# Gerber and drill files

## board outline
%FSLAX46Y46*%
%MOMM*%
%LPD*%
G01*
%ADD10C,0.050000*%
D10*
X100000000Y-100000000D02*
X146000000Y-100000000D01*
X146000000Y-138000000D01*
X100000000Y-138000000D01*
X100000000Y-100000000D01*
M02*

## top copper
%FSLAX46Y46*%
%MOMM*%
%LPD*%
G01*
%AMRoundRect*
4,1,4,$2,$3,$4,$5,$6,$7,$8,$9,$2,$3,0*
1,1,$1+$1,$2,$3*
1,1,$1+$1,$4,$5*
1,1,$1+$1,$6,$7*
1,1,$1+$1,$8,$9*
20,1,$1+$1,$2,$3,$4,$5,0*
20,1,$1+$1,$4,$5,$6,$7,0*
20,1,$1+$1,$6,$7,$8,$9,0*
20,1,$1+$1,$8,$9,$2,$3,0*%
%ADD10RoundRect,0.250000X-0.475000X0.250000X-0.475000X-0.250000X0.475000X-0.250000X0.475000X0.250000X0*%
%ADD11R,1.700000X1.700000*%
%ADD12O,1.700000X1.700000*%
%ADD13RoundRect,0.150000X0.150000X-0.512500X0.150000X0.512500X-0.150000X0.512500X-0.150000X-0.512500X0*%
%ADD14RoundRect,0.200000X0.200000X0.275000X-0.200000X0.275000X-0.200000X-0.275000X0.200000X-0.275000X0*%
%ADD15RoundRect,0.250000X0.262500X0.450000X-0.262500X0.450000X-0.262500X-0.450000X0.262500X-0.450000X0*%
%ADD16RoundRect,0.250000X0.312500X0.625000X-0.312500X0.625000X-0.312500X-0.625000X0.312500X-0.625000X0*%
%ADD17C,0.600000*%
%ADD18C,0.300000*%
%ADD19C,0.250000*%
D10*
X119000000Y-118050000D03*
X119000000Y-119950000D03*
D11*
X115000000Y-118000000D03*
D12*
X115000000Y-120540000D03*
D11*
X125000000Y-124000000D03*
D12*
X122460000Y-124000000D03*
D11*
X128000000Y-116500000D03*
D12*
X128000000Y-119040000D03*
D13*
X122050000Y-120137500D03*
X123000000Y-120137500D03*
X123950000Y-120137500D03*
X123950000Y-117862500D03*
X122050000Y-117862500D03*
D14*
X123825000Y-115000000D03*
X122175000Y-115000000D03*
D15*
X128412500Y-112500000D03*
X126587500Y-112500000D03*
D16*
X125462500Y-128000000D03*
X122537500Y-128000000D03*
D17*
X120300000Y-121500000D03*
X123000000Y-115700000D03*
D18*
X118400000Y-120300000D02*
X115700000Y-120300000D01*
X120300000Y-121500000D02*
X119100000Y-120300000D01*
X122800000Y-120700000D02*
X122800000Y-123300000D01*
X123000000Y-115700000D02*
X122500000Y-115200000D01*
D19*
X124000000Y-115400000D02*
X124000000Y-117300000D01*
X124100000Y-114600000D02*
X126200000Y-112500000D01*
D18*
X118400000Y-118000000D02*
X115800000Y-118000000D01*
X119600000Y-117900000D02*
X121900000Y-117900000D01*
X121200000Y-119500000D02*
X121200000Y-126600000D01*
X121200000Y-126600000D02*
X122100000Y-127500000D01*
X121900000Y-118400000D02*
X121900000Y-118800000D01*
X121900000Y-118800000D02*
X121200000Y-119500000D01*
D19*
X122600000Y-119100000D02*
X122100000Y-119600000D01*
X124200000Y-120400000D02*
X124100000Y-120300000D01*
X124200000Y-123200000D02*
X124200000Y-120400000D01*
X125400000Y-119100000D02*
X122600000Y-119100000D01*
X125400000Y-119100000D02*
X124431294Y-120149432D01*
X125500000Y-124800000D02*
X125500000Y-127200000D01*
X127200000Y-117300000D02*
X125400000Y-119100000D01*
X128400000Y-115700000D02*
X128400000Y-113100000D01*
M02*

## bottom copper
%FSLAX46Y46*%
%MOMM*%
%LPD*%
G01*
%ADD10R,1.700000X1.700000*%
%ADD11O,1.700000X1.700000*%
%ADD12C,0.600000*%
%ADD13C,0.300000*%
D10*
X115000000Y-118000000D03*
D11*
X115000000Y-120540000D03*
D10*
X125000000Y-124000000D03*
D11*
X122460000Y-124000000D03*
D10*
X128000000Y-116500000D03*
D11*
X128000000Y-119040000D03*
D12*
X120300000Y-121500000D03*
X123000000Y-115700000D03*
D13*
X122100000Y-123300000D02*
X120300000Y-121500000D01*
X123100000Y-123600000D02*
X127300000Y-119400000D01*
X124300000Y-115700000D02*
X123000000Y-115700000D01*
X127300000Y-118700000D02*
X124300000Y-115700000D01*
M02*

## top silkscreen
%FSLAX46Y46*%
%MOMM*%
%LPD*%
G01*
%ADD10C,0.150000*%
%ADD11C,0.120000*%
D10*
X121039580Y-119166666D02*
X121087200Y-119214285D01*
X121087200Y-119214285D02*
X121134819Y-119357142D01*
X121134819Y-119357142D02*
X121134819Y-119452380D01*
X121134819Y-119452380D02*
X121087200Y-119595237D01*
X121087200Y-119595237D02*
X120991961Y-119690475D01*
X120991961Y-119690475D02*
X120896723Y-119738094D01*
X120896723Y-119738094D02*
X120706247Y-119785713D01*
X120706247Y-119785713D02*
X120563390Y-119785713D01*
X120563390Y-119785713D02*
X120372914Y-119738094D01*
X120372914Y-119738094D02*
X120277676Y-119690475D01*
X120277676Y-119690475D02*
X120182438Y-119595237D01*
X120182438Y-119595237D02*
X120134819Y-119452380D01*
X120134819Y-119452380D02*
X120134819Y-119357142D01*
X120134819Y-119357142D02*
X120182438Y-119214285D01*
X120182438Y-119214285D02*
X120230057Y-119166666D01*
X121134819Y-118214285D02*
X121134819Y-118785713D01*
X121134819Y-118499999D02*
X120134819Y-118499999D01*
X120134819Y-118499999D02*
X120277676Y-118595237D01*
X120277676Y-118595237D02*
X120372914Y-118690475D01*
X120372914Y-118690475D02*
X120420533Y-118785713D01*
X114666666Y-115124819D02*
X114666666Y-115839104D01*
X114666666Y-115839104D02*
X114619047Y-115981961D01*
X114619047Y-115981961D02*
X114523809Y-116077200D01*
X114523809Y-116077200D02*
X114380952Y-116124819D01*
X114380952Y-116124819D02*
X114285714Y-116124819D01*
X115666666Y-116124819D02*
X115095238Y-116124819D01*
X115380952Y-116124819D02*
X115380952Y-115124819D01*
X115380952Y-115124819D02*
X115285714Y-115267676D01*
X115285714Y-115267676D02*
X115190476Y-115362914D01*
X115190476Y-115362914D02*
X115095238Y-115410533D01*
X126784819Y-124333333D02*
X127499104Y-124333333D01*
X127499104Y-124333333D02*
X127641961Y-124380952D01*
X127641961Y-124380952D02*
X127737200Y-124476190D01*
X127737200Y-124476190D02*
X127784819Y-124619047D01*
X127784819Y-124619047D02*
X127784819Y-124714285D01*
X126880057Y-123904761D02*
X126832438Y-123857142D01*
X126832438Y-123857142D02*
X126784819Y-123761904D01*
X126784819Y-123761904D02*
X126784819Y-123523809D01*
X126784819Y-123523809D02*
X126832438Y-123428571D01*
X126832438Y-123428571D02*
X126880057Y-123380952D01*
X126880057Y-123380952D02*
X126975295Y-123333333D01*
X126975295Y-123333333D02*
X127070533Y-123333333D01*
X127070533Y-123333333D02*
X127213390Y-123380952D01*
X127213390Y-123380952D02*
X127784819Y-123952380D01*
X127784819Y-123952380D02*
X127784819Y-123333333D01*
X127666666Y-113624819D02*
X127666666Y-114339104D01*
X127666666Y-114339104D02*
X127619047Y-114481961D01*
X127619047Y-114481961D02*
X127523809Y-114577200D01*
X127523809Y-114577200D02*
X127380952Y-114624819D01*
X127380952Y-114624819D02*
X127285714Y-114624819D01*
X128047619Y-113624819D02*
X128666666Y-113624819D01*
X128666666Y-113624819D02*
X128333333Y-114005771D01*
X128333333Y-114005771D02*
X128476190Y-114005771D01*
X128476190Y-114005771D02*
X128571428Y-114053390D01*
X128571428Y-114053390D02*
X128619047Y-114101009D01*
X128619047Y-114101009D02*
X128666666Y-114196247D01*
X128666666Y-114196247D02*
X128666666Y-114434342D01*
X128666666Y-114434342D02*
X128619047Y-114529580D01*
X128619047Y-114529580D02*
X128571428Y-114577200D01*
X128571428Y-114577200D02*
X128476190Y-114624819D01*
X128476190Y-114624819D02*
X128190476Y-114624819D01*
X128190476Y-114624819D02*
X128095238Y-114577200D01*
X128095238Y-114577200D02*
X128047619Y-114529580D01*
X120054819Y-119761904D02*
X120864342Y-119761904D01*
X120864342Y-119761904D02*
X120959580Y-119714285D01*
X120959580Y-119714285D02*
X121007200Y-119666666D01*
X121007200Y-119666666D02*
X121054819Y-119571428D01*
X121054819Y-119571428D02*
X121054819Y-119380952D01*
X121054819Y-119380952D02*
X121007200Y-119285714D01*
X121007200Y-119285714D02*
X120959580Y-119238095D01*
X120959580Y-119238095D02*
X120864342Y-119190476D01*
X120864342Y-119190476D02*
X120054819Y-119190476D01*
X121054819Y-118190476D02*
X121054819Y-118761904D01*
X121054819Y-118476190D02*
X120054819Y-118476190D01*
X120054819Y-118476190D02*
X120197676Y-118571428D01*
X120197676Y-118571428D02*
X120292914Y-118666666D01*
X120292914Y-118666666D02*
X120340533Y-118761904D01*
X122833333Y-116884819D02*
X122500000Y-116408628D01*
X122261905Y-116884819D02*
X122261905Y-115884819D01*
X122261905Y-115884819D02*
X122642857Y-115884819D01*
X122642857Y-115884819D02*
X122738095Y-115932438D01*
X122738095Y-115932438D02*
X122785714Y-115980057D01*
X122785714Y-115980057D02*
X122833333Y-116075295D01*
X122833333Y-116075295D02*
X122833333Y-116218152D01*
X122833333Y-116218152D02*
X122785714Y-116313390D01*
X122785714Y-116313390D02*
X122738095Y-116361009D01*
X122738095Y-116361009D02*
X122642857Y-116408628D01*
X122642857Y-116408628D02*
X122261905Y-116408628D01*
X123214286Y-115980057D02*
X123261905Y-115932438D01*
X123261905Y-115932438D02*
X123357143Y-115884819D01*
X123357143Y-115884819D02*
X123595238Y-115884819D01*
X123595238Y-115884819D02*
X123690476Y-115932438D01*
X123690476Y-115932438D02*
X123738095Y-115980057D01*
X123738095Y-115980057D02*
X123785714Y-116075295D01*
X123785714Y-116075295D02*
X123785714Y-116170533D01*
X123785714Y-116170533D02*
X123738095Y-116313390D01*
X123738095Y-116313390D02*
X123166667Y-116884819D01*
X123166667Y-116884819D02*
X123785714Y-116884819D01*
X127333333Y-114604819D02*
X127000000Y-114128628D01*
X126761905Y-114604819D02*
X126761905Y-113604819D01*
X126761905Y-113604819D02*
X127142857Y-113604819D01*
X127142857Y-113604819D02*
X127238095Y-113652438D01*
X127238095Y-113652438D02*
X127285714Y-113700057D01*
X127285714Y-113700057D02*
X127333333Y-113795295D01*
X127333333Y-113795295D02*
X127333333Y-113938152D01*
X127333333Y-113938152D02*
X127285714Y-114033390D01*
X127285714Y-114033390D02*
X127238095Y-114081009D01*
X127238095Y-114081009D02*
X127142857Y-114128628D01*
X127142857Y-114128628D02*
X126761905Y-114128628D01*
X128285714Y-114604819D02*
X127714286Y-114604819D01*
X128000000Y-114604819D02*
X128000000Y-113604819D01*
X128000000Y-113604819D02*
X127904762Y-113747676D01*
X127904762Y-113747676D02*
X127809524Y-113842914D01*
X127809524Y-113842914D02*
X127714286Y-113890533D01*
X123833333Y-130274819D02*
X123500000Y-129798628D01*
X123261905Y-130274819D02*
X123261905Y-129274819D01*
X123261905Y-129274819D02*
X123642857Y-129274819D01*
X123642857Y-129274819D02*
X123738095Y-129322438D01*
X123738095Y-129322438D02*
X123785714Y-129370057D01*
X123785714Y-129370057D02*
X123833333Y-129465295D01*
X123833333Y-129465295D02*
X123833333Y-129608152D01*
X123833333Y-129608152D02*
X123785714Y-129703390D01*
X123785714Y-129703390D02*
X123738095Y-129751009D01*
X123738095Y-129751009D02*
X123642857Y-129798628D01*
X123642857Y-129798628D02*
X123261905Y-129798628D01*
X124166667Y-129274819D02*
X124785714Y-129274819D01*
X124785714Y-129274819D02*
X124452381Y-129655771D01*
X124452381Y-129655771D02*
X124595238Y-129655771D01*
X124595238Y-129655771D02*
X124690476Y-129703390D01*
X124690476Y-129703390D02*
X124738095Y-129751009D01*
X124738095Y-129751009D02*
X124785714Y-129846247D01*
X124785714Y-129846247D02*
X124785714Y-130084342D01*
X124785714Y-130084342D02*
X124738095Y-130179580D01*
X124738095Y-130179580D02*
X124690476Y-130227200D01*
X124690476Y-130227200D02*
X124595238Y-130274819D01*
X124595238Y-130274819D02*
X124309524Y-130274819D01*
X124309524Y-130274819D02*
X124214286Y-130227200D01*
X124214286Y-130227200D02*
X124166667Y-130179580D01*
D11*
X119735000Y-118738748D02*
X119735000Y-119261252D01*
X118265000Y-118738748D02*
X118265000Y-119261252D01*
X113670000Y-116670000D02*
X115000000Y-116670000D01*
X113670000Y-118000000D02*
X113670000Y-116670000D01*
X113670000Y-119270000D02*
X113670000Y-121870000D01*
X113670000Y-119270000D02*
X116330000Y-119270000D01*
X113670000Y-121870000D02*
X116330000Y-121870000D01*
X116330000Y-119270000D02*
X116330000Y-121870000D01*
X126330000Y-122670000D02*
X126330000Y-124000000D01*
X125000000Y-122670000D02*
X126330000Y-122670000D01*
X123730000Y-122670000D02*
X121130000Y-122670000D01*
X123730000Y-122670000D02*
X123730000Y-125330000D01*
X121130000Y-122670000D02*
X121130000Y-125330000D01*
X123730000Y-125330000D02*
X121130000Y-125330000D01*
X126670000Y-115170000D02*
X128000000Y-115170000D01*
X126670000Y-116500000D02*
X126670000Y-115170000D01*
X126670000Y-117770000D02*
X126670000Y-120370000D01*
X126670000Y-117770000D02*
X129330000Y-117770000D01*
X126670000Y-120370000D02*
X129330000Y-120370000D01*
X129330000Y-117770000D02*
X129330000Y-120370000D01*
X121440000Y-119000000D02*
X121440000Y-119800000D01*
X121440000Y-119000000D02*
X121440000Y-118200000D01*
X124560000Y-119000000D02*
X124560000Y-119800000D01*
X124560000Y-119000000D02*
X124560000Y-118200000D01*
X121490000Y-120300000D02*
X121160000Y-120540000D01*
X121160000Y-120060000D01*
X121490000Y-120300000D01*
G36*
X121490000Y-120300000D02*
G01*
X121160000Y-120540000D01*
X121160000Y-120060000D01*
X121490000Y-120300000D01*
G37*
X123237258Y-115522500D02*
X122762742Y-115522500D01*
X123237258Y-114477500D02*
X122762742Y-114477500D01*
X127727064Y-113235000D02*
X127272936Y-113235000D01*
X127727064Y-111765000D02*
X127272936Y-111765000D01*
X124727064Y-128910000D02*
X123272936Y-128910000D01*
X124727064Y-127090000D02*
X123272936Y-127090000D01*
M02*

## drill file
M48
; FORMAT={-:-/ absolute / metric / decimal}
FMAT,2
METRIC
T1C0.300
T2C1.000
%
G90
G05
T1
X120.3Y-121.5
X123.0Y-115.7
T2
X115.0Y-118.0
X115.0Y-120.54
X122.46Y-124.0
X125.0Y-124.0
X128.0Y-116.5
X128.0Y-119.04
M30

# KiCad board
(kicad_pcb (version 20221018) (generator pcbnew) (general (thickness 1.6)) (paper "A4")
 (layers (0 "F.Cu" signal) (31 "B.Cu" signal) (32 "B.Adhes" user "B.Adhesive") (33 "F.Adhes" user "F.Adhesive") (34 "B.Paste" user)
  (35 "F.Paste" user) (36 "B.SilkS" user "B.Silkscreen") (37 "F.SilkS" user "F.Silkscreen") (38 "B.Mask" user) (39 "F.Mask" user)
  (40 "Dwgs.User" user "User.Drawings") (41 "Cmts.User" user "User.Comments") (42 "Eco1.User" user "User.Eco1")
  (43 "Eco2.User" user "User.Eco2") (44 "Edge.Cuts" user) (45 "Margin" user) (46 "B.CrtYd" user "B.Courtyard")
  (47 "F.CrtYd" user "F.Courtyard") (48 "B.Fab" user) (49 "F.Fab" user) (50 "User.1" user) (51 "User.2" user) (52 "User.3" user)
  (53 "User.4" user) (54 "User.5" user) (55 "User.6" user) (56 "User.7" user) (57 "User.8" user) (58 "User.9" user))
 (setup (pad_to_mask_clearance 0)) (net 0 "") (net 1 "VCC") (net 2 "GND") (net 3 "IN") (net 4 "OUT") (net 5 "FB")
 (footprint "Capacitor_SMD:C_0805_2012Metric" (layer "F.Cu") (at 119 119 -90)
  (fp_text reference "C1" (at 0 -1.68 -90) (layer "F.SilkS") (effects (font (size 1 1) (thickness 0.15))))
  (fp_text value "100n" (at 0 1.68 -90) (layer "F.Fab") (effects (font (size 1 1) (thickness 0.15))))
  (fp_line (start -0.261252 -0.735) (end 0.261252 -0.735) (stroke (width 0.12) (type solid)) (layer "F.SilkS"))
  (fp_line (start -0.261252 0.735) (end 0.261252 0.735) (stroke (width 0.12) (type solid)) (layer "F.SilkS"))
  (pad "1" smd roundrect (at -0.95 0 270) (size 1 1.45) (layers "F.Cu" "F.Paste" "F.Mask") (roundrect_rratio 0.25) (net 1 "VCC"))
  (pad "2" smd roundrect (at 0.95 0 270) (size 1 1.45) (layers "F.Cu" "F.Paste" "F.Mask") (roundrect_rratio 0.25) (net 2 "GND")))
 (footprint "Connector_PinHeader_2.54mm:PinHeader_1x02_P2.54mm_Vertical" (layer "F.Cu") (at 115 118)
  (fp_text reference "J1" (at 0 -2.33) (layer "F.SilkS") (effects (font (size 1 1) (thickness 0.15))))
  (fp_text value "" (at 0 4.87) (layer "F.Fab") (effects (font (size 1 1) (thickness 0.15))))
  (fp_line (start -1.33 -1.33) (end 0 -1.33) (stroke (width 0.12) (type solid)) (layer "F.SilkS"))
  (fp_line (start -1.33 0) (end -1.33 -1.33) (stroke (width 0.12) (type solid)) (layer "F.SilkS"))
  (fp_line (start -1.33 1.27) (end -1.33 3.87) (stroke (width 0.12) (type solid)) (layer "F.SilkS"))
  (fp_line (start -1.33 1.27) (end 1.33 1.27) (stroke (width 0.12) (type solid)) (layer "F.SilkS"))
  (fp_line (start -1.33 3.87) (end 1.33 3.87) (stroke (width 0.12) (type solid)) (layer "F.SilkS"))
  (fp_line (start 1.33 1.27) (end 1.33 3.87) (stroke (width 0.12) (type solid)) (layer "F.SilkS"))
  (pad "1" thru_hole rect (at 0 0) (size 1.7 1.7) (drill 1) (layers "*.Cu" "*.Mask") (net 1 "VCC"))
  (pad "2" thru_hole oval (at 0 2.54) (size 1.7 1.7) (drill 1) (layers "*.Cu" "*.Mask") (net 2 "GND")))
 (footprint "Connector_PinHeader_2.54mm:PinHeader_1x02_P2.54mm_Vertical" (layer "F.Cu") (at 125 124 -90)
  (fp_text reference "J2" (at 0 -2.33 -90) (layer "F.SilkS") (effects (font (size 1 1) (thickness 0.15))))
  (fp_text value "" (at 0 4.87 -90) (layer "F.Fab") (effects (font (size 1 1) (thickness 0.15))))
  (fp_line (start -1.33 -1.33) (end 0 -1.33) (stroke (width 0.12) (type solid)) (layer "F.SilkS"))
  (fp_line (start -1.33 0) (end -1.33 -1.33) (stroke (width 0.12) (type solid)) (layer "F.SilkS"))
  (fp_line (start -1.33 1.27) (end -1.33 3.87) (stroke (width 0.12) (type solid)) (layer "F.SilkS"))
  (fp_line (start -1.33 1.27) (end 1.33 1.27) (stroke (width 0.12) (type solid)) (layer "F.SilkS"))
  (fp_line (start -1.33 3.87) (end 1.33 3.87) (stroke (width 0.12) (type solid)) (layer "F.SilkS"))
  (fp_line (start 1.33 1.27) (end 1.33 3.87) (stroke (width 0.12) (type solid)) (layer "F.SilkS"))
  (pad "1" thru_hole rect (at 0 0 270) (size 1.7 1.7) (drill 1) (layers "*.Cu" "*.Mask") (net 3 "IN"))
  (pad "2" thru_hole oval (at 0 2.54 270) (size 1.7 1.7) (drill 1) (layers "*.Cu" "*.Mask") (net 2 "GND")))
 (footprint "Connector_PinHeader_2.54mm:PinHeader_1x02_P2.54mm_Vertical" (layer "F.Cu") (at 128 116.5)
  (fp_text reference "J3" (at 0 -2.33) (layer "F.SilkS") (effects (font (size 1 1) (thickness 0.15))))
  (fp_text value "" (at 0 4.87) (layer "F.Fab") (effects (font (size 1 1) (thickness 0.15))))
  (fp_line (start -1.33 -1.33) (end 0 -1.33) (stroke (width 0.12) (type solid)) (layer "F.SilkS"))
  (fp_line (start -1.33 0) (end -1.33 -1.33) (stroke (width 0.12) (type solid)) (layer "F.SilkS"))
  (fp_line (start -1.33 1.27) (end -1.33 3.87) (stroke (width 0.12) (type solid)) (layer "F.SilkS"))
  (fp_line (start -1.33 1.27) (end 1.33 1.27) (stroke (width 0.12) (type solid)) (layer "F.SilkS"))
  (fp_line (start -1.33 3.87) (end 1.33 3.87) (stroke (width 0.12) (type solid)) (layer "F.SilkS"))
  (fp_line (start 1.33 1.27) (end 1.33 3.87) (stroke (width 0.12) (type solid)) (layer "F.SilkS"))
  (pad "1" thru_hole rect (at 0 0) (size 1.7 1.7) (drill 1) (layers "*.Cu" "*.Mask") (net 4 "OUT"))
  (pad "2" thru_hole oval (at 0 2.54) (size 1.7 1.7) (drill 1) (layers "*.Cu" "*.Mask") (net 2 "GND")))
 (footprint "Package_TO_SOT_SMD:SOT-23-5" (layer "F.Cu") (at 123 119 90)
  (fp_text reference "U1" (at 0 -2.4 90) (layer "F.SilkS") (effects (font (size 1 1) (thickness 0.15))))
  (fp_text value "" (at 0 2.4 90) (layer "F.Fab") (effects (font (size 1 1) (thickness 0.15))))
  (fp_line (start 0 -1.56) (end -0.8 -1.56) (stroke (width 0.12) (type solid)) (layer "F.SilkS"))
  (fp_line (start 0 -1.56) (end 0.8 -1.56) (stroke (width 0.12) (type solid)) (layer "F.SilkS"))
  (fp_line (start 0 1.56) (end -0.8 1.56) (stroke (width 0.12) (type solid)) (layer "F.SilkS"))
  (fp_line (start 0 1.56) (end 0.8 1.56) (stroke (width 0.12) (type solid)) (layer "F.SilkS"))
  (fp_poly
   (pts (xy -1.3 -1.51) (xy -1.54 -1.84) (xy -1.06 -1.84) (xy -1.3 -1.51)) (stroke (width 0.12) (type solid)) (fill solid) (layer "F.SilkS"))
  (pad "1" smd roundrect (at -1.1375 -0.95 90) (size 1.325 0.6) (layers "F.Cu" "F.Paste" "F.Mask") (roundrect_rratio 0.25) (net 4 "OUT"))
  (pad "2" smd roundrect (at -1.1375 0 90) (size 1.325 0.6) (layers "F.Cu" "F.Paste" "F.Mask") (roundrect_rratio 0.25) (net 2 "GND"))
  (pad "3" smd roundrect (at -1.1375 0.95 90) (size 1.325 0.6) (layers "F.Cu" "F.Paste" "F.Mask") (roundrect_rratio 0.25) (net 3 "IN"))
  (pad "4" smd roundrect (at 1.1375 0.95 90) (size 1.325 0.6) (layers "F.Cu" "F.Paste" "F.Mask") (roundrect_rratio 0.25) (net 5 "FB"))
  (pad "5" smd roundrect (at 1.1375 -0.95 90) (size 1.325 0.6) (layers "F.Cu" "F.Paste" "F.Mask") (roundrect_rratio 0.25) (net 1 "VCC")))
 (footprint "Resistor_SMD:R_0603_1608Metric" (layer "F.Cu") (at 123 115 180)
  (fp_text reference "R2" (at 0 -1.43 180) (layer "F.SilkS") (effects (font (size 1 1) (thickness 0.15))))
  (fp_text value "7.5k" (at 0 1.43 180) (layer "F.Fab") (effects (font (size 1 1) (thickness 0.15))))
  (fp_line (start -0.237258 -0.5225) (end 0.237258 -0.5225) (stroke (width 0.12) (type solid)) (layer "F.SilkS"))
  (fp_line (start -0.237258 0.5225) (end 0.237258 0.5225) (stroke (width 0.12) (type solid)) (layer "F.SilkS"))
  (pad "1" smd roundrect (at -0.825 0 180) (size 0.8 0.95) (layers "F.Cu" "F.Paste" "F.Mask") (roundrect_rratio 0.25) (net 5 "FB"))
  (pad "2" smd roundrect (at 0.825 0 180) (size 0.8 0.95) (layers "F.Cu" "F.Paste" "F.Mask") (roundrect_rratio 0.25) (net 2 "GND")))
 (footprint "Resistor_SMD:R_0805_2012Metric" (layer "F.Cu") (at 127.5 112.5 180)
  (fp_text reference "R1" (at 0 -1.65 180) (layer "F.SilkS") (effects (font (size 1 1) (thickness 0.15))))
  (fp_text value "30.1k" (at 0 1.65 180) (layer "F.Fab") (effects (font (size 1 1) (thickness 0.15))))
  (fp_line (start -0.227064 -0.735) (end 0.227064 -0.735) (stroke (width 0.12) (type solid)) (layer "F.SilkS"))
  (fp_line (start -0.227064 0.735) (end 0.227064 0.735) (stroke (width 0.12) (type solid)) (layer "F.SilkS"))
  (pad "1" smd roundrect (at -0.9125 0 180) (size 1.025 1.4) (layers "F.Cu" "F.Paste" "F.Mask") (roundrect_rratio 0.243902) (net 4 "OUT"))
  (pad "2" smd roundrect (at 0.9125 0 180) (size 1.025 1.4) (layers "F.Cu" "F.Paste" "F.Mask") (roundrect_rratio 0.243902) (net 5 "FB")))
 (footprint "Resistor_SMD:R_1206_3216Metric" (layer "F.Cu") (at 124 128 180)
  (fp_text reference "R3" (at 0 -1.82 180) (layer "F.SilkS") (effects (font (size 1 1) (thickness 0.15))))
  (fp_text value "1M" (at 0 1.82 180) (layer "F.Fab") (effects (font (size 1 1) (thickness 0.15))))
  (fp_line (start -0.727064 -0.91) (end 0.727064 -0.91) (stroke (width 0.12) (type solid)) (layer "F.SilkS"))
  (fp_line (start -0.727064 0.91) (end 0.727064 0.91) (stroke (width 0.12) (type solid)) (layer "F.SilkS"))
  (pad "1" smd roundrect (at -1.4625 0 180) (size 1.125 1.75) (layers "F.Cu" "F.Paste" "F.Mask") (roundrect_rratio 0.222222) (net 3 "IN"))
  (pad "2" smd roundrect (at 1.4625 0 180) (size 1.125 1.75) (layers "F.Cu" "F.Paste" "F.Mask") (roundrect_rratio 0.222222) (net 1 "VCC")))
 (gr_rect (start 100 100) (end 146 138) (stroke (width 0.05) (type default)) (fill none) (layer "Edge.Cuts"))
 (segment (start 118.4 120.3) (end 115.7 120.3) (width 0.3) (layer "F.Cu") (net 2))
 (segment (start 120.3 121.5) (end 119.1 120.3) (width 0.3) (layer "F.Cu") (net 2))
 (segment (start 122.8 120.7) (end 122.8 123.3) (width 0.3) (layer "F.Cu") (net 2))
 (segment (start 123 115.7) (end 122.5 115.2) (width 0.3) (layer "F.Cu") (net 2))
 (segment (start 124 115.4) (end 124 117.3) (width 0.25) (layer "F.Cu") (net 5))
 (segment (start 124.1 114.6) (end 126.2 112.5) (width 0.25) (layer "F.Cu") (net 5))
 (via (at 120.3 121.5) (size 0.6) (drill 0.3) (layers "F.Cu" "B.Cu") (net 2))
 (via (at 123 115.7) (size 0.6) (drill 0.3) (layers "F.Cu" "B.Cu") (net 2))
 (segment (start 118.4 118) (end 115.8 118) (width 0.3) (layer "F.Cu") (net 1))
 (segment (start 119.6 117.9) (end 121.9 117.9) (width 0.3) (layer "F.Cu") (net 1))
 (segment (start 121.2 119.5) (end 121.2 126.6) (width 0.3) (layer "F.Cu") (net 1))
 (segment (start 121.2 126.6) (end 122.1 127.5) (width 0.3) (layer "F.Cu") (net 1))
 (segment (start 121.9 118.4) (end 121.9 118.8) (width 0.3) (layer "F.Cu") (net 1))
 (segment (start 121.9 118.8) (end 121.2 119.5) (width 0.3) (layer "F.Cu") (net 1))
 (segment (start 122.1 123.3) (end 120.3 121.5) (width 0.3) (layer "B.Cu") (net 2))
 (segment (start 122.6 119.1) (end 122.1 119.6) (width 0.25) (layer "F.Cu") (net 4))
 (segment (start 123.1 123.6) (end 127.3 119.4) (width 0.3) (layer "B.Cu") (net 2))
 (segment (start 124.2 120.4) (end 124.1 120.3) (width 0.25) (layer "F.Cu") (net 3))
 (segment (start 124.2 123.2) (end 124.2 120.4) (width 0.25) (layer "F.Cu") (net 3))
 (segment (start 124.3 115.7) (end 123 115.7) (width 0.3) (layer "B.Cu") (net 2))
 (segment (start 125.4 119.1) (end 122.6 119.1) (width 0.25) (layer "F.Cu") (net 4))
 (segment (start 125.4 119.1) (end 124.431294 120.149432) (width 0.25) (layer "F.Cu") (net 4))
 (segment (start 125.5 124.8) (end 125.5 127.2) (width 0.25) (layer "F.Cu") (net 3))
 (segment (start 127.2 117.3) (end 125.4 119.1) (width 0.25) (layer "F.Cu") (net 4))
 (segment (start 127.3 118.7) (end 124.3 115.7) (width 0.3) (layer "B.Cu") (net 2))
 (segment (start 128.4 115.7) (end 128.4 113.1) (width 0.25) (layer "F.Cu") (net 4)))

